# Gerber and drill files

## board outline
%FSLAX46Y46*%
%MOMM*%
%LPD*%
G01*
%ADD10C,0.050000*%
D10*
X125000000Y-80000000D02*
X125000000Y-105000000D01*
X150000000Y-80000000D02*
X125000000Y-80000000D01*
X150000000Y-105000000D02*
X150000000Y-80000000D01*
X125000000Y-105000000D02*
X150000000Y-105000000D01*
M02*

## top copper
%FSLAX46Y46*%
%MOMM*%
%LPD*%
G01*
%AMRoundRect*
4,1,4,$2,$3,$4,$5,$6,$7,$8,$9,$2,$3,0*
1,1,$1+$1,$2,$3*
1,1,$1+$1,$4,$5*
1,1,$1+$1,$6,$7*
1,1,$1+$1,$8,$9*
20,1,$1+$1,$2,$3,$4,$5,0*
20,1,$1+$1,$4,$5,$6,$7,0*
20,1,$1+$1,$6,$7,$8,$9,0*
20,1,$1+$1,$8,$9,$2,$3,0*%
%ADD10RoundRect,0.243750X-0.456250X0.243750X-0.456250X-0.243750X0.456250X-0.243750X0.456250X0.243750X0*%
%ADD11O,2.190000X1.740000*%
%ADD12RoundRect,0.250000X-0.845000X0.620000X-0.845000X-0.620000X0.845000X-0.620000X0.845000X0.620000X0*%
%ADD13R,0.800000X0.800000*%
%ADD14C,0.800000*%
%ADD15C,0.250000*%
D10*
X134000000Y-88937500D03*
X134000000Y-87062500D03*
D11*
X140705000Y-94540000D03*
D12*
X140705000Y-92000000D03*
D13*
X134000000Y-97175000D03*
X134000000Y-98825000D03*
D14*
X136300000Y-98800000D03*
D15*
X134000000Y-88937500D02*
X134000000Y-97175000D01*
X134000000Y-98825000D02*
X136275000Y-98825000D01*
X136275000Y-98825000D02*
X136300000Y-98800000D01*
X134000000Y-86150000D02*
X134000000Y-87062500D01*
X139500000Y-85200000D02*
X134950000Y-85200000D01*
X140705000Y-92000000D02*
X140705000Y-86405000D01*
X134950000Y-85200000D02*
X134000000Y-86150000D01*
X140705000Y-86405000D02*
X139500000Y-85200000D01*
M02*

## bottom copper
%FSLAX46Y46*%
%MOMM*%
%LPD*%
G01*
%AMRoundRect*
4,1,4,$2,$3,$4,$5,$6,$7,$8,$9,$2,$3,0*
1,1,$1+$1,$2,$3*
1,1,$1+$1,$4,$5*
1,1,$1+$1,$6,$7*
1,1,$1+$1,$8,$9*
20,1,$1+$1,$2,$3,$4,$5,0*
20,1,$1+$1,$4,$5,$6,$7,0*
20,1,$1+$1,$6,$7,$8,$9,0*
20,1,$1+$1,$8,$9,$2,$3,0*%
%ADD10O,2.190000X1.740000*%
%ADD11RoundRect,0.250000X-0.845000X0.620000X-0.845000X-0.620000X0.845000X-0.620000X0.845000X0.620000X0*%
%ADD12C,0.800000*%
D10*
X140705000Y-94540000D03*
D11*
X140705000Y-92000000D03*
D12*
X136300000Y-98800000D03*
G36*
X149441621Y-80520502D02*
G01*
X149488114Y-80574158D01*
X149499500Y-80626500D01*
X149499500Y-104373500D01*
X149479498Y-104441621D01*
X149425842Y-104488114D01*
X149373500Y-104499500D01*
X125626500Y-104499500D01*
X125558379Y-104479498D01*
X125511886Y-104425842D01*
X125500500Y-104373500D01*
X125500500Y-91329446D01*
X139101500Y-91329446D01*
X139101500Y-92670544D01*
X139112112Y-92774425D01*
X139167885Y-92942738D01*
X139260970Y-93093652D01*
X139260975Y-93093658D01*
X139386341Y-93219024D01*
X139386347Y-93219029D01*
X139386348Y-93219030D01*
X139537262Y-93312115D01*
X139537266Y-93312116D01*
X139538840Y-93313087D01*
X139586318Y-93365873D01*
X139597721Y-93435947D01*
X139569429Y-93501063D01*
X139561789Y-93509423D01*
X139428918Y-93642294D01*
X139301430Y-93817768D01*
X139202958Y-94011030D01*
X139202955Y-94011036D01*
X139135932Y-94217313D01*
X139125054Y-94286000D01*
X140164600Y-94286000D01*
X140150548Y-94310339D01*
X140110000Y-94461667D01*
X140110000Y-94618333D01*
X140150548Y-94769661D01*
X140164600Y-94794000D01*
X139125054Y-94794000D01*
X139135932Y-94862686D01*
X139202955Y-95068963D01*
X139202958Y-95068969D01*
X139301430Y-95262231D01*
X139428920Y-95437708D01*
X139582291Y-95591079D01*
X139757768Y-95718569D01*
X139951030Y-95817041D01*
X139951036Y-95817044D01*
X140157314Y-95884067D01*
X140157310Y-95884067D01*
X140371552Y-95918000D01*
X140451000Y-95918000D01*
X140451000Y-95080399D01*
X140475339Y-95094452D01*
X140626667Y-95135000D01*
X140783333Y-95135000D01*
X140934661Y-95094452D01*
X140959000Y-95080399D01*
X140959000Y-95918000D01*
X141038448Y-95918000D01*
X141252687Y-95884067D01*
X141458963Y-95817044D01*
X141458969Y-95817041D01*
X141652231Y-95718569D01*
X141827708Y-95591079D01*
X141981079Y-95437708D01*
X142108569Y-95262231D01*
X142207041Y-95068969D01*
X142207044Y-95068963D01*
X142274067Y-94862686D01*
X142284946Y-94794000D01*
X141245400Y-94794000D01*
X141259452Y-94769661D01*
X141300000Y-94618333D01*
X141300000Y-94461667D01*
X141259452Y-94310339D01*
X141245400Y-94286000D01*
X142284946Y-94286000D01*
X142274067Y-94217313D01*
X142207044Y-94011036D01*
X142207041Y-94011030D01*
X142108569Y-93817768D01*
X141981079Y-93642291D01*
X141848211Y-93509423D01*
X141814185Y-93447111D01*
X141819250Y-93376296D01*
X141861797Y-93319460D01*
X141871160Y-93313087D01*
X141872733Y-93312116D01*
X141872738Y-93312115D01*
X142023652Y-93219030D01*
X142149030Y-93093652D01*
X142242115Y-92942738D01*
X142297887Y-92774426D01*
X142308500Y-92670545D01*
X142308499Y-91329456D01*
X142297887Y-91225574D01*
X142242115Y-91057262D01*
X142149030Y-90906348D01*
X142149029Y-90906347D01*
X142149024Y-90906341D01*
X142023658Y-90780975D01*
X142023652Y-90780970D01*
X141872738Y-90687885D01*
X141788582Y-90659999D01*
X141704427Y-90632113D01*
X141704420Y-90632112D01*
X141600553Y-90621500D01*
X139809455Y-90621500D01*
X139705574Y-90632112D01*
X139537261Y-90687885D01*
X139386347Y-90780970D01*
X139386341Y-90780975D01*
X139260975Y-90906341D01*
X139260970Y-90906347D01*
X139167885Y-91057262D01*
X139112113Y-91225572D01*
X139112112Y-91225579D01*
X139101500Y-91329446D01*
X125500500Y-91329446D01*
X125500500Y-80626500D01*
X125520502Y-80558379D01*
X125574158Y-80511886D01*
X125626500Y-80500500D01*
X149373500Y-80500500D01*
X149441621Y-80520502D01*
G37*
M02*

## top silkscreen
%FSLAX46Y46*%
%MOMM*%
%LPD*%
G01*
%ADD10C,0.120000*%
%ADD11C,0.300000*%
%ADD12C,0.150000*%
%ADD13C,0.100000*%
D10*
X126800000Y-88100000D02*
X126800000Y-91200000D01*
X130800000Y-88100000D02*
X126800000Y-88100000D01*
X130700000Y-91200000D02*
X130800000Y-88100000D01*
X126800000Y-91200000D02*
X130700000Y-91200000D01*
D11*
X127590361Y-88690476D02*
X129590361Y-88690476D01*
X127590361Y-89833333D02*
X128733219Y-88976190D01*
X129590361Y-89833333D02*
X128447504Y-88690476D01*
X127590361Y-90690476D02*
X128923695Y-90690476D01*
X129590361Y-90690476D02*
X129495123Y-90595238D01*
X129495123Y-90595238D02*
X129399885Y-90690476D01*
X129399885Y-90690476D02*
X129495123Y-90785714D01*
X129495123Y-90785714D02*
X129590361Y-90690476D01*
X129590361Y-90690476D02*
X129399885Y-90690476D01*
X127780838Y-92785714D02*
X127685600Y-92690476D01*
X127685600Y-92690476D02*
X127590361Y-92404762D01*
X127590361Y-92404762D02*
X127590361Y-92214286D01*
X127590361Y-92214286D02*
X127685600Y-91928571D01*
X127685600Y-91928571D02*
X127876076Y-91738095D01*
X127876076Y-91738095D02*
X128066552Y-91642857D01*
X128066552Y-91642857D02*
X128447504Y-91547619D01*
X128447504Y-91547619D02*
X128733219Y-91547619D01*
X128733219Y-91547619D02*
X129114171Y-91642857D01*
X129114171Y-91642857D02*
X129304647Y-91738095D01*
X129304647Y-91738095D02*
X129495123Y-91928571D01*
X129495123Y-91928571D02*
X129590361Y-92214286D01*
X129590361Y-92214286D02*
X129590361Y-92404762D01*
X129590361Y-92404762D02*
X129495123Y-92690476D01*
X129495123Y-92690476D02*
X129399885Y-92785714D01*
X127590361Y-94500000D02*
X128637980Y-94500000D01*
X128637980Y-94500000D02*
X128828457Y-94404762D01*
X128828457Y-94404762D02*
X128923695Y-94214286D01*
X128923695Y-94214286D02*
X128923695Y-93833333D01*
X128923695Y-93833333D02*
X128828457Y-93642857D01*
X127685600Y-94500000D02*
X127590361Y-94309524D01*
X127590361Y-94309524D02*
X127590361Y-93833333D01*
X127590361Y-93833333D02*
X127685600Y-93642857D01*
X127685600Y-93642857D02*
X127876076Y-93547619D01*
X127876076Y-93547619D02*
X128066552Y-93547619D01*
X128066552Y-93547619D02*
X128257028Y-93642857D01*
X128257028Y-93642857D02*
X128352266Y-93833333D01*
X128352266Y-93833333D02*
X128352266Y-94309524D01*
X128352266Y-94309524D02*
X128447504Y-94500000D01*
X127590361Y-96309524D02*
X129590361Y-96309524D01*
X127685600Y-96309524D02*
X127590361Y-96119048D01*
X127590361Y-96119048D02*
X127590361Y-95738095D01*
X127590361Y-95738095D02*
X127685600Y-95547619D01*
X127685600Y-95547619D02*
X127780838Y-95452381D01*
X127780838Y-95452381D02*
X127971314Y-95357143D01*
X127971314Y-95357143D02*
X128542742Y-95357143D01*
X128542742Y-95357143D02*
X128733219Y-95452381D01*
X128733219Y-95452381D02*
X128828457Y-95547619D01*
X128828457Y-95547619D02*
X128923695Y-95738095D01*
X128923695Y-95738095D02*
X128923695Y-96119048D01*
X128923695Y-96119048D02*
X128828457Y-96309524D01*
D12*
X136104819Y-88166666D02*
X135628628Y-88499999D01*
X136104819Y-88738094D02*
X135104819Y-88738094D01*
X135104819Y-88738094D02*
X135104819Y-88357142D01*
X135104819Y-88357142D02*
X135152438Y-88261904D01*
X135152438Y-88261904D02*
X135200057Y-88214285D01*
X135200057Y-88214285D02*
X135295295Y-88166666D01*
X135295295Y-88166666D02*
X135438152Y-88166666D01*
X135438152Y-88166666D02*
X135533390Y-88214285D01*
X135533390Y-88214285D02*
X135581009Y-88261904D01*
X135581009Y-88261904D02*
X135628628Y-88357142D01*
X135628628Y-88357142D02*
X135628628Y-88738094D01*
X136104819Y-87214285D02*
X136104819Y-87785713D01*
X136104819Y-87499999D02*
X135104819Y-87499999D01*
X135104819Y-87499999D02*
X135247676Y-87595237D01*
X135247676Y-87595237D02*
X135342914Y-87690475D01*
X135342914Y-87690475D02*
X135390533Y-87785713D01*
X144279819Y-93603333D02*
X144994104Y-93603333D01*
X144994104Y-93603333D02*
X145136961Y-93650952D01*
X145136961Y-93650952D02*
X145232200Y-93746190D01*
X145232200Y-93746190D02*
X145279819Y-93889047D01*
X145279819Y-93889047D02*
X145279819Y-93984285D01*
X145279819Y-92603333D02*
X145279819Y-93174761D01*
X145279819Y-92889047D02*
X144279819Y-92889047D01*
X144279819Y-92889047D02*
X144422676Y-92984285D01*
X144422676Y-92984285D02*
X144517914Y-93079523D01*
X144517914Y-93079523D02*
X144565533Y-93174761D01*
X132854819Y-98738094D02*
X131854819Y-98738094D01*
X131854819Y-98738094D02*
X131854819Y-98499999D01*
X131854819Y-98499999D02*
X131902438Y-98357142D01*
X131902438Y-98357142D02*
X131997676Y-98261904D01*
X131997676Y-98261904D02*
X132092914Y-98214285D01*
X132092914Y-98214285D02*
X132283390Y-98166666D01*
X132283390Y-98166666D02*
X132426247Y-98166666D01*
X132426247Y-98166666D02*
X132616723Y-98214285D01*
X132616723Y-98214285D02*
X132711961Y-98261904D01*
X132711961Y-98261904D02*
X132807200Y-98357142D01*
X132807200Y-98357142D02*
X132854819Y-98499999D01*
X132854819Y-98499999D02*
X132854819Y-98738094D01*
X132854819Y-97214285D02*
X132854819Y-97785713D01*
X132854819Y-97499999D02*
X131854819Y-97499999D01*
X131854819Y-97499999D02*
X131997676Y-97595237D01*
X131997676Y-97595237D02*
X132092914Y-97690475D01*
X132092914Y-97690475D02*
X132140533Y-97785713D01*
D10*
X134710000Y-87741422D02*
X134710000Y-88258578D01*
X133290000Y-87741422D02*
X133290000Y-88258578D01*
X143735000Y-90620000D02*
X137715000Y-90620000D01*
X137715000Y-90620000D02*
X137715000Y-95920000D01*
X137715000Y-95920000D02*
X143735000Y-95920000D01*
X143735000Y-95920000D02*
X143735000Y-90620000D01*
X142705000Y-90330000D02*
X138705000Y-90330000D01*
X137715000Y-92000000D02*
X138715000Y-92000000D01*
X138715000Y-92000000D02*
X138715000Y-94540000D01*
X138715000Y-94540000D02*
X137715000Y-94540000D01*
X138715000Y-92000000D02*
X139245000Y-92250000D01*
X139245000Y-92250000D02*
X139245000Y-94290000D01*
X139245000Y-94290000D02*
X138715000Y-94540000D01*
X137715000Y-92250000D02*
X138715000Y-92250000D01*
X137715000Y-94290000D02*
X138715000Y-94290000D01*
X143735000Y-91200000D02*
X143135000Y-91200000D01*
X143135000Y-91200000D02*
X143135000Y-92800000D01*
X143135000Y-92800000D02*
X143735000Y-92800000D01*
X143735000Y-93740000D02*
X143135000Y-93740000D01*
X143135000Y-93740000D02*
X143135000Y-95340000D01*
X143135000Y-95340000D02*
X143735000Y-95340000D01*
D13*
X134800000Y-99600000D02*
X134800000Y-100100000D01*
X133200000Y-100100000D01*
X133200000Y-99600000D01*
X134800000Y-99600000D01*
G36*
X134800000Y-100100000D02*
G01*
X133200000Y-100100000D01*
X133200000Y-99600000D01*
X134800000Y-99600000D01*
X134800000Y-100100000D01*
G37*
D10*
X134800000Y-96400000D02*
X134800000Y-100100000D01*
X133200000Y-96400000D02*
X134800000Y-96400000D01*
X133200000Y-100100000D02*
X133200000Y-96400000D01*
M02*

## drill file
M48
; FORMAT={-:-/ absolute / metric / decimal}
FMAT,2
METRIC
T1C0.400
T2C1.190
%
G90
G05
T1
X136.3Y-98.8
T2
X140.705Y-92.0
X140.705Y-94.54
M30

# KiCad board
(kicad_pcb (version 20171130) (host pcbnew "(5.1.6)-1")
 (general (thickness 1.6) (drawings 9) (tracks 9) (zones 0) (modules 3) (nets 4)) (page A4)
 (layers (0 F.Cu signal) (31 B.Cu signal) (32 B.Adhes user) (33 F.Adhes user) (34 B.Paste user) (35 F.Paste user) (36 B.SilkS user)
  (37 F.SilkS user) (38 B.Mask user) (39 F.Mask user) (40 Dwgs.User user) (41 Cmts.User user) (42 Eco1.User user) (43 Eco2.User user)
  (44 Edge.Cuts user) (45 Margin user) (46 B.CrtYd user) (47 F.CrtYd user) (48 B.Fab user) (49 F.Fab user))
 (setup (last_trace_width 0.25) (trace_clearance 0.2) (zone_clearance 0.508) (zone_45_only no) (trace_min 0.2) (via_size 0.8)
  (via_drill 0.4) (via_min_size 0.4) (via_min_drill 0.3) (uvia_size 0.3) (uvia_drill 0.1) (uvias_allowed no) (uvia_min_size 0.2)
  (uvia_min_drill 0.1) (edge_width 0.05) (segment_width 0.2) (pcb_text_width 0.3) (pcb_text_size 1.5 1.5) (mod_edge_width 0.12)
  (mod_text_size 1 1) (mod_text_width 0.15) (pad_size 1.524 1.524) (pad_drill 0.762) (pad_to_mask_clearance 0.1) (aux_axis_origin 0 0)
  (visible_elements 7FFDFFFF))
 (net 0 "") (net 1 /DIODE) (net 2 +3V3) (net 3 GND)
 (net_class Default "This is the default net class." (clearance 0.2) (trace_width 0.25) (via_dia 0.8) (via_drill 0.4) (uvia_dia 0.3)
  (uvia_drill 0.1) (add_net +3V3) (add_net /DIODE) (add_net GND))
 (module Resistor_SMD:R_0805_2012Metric (layer F.Cu) (at 134 88 270)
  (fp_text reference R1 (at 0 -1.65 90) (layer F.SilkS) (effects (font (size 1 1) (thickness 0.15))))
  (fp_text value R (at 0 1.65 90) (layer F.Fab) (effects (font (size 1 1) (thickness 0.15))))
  (fp_line (start -0.258578 -0.71) (end 0.258578 -0.71) (layer F.SilkS) (width 0.12))
  (fp_line (start -0.258578 0.71) (end 0.258578 0.71) (layer F.SilkS) (width 0.12))
  (pad 2 smd roundrect (at 0.9375 0 270) (size 0.975 1.4) (layers F.Cu F.Paste F.Mask) (roundrect_rratio 0.25) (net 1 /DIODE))
  (pad 1 smd roundrect (at -0.9375 0 270) (size 0.975 1.4) (layers F.Cu F.Paste F.Mask) (roundrect_rratio 0.25) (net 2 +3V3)))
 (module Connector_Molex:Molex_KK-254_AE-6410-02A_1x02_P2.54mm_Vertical (layer F.Cu) (at 140.705 92 270)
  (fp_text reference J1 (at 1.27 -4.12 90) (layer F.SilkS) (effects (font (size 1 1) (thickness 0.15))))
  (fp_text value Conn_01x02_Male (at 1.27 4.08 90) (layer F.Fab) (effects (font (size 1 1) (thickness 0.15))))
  (fp_line (start -1.38 -3.03) (end -1.38 2.99) (layer F.SilkS) (width 0.12))
  (fp_line (start -1.38 2.99) (end 3.92 2.99) (layer F.SilkS) (width 0.12))
  (fp_line (start 3.92 2.99) (end 3.92 -3.03) (layer F.SilkS) (width 0.12))
  (fp_line (start 3.92 -3.03) (end -1.38 -3.03) (layer F.SilkS) (width 0.12))
  (fp_line (start -1.67 -2) (end -1.67 2) (layer F.SilkS) (width 0.12))
  (fp_line (start 0 2.99) (end 0 1.99) (layer F.SilkS) (width 0.12))
  (fp_line (start 0 1.99) (end 2.54 1.99) (layer F.SilkS) (width 0.12))
  (fp_line (start 2.54 1.99) (end 2.54 2.99) (layer F.SilkS) (width 0.12))
  (fp_line (start 0 1.99) (end 0.25 1.46) (layer F.SilkS) (width 0.12))
  (fp_line (start 0.25 1.46) (end 2.29 1.46) (layer F.SilkS) (width 0.12))
  (fp_line (start 2.29 1.46) (end 2.54 1.99) (layer F.SilkS) (width 0.12))
  (fp_line (start 0.25 2.99) (end 0.25 1.99) (layer F.SilkS) (width 0.12))
  (fp_line (start 2.29 2.99) (end 2.29 1.99) (layer F.SilkS) (width 0.12))
  (fp_line (start -0.8 -3.03) (end -0.8 -2.43) (layer F.SilkS) (width 0.12))
  (fp_line (start -0.8 -2.43) (end 0.8 -2.43) (layer F.SilkS) (width 0.12))
  (fp_line (start 0.8 -2.43) (end 0.8 -3.03) (layer F.SilkS) (width 0.12))
  (fp_line (start 1.74 -3.03) (end 1.74 -2.43) (layer F.SilkS) (width 0.12))
  (fp_line (start 1.74 -2.43) (end 3.34 -2.43) (layer F.SilkS) (width 0.12))
  (fp_line (start 3.34 -2.43) (end 3.34 -3.03) (layer F.SilkS) (width 0.12))
  (pad 2 thru_hole oval (at 2.54 0 270) (size 1.74 2.19) (drill 1.19) (layers *.Cu *.Mask) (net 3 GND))
  (pad 1 thru_hole roundrect (at 0 0 270) (size 1.74 2.19) (drill 1.19) (layers *.Cu *.Mask) (roundrect_rratio 0.143678) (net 2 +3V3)))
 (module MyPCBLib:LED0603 (layer F.Cu) (at 134 98 90)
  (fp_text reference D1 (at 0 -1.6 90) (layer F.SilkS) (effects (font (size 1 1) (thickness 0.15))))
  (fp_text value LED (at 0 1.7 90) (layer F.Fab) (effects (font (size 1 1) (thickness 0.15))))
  (fp_poly (pts (xy -1.6 0.8) (xy -2.1 0.8) (xy -2.1 -0.8) (xy -1.6 -0.8)) (layer F.SilkS) (width 0.1))
  (fp_line (start 1.6 0.8) (end -2.1 0.8) (layer F.SilkS) (width 0.12))
  (fp_line (start 1.6 -0.8) (end 1.6 0.8) (layer F.SilkS) (width 0.12))
  (fp_line (start -2.1 -0.8) (end 1.6 -0.8) (layer F.SilkS) (width 0.12))
  (pad A smd rect (at 0.825 0 90) (size 0.8 0.8) (layers F.Cu F.Paste F.Mask) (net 1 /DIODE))
  (pad C smd rect (at -0.825 0 90) (size 0.8 0.8) (layers F.Cu F.Paste F.Mask) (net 3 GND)))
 (gr_line (start 126.8 88.1) (end 126.8 91.2) (layer F.SilkS) (width 0.12))
 (gr_line (start 130.8 88.1) (end 126.8 88.1) (layer F.SilkS) (width 0.12))
 (gr_line (start 130.7 91.2) (end 130.8 88.1) (layer F.SilkS) (width 0.12))
 (gr_line (start 126.8 91.2) (end 130.7 91.2) (layer F.SilkS) (width 0.12))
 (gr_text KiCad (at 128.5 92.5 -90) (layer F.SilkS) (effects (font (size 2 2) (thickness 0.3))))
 (gr_line (start 125 80) (end 125 105) (layer Edge.Cuts) (width 0.05))
 (gr_line (start 150 80) (end 125 80) (layer Edge.Cuts) (width 0.05))
 (gr_line (start 150 105) (end 150 80) (layer Edge.Cuts) (width 0.05))
 (gr_line (start 125 105) (end 150 105) (layer Edge.Cuts) (width 0.05))
 (segment (start 134 88.9375) (end 134 97.175) (width 0.25) (layer F.Cu) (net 1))
 (via (at 136.3 98.8) (size 0.8) (drill 0.4) (layers F.Cu B.Cu) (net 3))
 (segment (start 134 98.825) (end 136.275 98.825) (width 0.25) (layer F.Cu) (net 3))
 (segment (start 136.275 98.825) (end 136.3 98.8) (width 0.25) (layer F.Cu) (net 3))
 (segment (start 134 86.15) (end 134 87.0625) (width 0.25) (layer F.Cu) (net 2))
 (segment (start 139.5 85.2) (end 134.95 85.2) (width 0.25) (layer F.Cu) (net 2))
 (segment (start 140.705 92) (end 140.705 86.405) (width 0.25) (layer F.Cu) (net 2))
 (segment (start 134.95 85.2) (end 134 86.15) (width 0.25) (layer F.Cu) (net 2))
 (segment (start 140.705 86.405) (end 139.5 85.2) (width 0.25) (layer F.Cu) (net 2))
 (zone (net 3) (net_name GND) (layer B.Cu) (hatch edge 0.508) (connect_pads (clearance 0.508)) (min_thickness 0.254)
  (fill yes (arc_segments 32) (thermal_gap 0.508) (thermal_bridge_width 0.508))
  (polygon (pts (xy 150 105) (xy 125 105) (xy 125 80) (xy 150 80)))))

